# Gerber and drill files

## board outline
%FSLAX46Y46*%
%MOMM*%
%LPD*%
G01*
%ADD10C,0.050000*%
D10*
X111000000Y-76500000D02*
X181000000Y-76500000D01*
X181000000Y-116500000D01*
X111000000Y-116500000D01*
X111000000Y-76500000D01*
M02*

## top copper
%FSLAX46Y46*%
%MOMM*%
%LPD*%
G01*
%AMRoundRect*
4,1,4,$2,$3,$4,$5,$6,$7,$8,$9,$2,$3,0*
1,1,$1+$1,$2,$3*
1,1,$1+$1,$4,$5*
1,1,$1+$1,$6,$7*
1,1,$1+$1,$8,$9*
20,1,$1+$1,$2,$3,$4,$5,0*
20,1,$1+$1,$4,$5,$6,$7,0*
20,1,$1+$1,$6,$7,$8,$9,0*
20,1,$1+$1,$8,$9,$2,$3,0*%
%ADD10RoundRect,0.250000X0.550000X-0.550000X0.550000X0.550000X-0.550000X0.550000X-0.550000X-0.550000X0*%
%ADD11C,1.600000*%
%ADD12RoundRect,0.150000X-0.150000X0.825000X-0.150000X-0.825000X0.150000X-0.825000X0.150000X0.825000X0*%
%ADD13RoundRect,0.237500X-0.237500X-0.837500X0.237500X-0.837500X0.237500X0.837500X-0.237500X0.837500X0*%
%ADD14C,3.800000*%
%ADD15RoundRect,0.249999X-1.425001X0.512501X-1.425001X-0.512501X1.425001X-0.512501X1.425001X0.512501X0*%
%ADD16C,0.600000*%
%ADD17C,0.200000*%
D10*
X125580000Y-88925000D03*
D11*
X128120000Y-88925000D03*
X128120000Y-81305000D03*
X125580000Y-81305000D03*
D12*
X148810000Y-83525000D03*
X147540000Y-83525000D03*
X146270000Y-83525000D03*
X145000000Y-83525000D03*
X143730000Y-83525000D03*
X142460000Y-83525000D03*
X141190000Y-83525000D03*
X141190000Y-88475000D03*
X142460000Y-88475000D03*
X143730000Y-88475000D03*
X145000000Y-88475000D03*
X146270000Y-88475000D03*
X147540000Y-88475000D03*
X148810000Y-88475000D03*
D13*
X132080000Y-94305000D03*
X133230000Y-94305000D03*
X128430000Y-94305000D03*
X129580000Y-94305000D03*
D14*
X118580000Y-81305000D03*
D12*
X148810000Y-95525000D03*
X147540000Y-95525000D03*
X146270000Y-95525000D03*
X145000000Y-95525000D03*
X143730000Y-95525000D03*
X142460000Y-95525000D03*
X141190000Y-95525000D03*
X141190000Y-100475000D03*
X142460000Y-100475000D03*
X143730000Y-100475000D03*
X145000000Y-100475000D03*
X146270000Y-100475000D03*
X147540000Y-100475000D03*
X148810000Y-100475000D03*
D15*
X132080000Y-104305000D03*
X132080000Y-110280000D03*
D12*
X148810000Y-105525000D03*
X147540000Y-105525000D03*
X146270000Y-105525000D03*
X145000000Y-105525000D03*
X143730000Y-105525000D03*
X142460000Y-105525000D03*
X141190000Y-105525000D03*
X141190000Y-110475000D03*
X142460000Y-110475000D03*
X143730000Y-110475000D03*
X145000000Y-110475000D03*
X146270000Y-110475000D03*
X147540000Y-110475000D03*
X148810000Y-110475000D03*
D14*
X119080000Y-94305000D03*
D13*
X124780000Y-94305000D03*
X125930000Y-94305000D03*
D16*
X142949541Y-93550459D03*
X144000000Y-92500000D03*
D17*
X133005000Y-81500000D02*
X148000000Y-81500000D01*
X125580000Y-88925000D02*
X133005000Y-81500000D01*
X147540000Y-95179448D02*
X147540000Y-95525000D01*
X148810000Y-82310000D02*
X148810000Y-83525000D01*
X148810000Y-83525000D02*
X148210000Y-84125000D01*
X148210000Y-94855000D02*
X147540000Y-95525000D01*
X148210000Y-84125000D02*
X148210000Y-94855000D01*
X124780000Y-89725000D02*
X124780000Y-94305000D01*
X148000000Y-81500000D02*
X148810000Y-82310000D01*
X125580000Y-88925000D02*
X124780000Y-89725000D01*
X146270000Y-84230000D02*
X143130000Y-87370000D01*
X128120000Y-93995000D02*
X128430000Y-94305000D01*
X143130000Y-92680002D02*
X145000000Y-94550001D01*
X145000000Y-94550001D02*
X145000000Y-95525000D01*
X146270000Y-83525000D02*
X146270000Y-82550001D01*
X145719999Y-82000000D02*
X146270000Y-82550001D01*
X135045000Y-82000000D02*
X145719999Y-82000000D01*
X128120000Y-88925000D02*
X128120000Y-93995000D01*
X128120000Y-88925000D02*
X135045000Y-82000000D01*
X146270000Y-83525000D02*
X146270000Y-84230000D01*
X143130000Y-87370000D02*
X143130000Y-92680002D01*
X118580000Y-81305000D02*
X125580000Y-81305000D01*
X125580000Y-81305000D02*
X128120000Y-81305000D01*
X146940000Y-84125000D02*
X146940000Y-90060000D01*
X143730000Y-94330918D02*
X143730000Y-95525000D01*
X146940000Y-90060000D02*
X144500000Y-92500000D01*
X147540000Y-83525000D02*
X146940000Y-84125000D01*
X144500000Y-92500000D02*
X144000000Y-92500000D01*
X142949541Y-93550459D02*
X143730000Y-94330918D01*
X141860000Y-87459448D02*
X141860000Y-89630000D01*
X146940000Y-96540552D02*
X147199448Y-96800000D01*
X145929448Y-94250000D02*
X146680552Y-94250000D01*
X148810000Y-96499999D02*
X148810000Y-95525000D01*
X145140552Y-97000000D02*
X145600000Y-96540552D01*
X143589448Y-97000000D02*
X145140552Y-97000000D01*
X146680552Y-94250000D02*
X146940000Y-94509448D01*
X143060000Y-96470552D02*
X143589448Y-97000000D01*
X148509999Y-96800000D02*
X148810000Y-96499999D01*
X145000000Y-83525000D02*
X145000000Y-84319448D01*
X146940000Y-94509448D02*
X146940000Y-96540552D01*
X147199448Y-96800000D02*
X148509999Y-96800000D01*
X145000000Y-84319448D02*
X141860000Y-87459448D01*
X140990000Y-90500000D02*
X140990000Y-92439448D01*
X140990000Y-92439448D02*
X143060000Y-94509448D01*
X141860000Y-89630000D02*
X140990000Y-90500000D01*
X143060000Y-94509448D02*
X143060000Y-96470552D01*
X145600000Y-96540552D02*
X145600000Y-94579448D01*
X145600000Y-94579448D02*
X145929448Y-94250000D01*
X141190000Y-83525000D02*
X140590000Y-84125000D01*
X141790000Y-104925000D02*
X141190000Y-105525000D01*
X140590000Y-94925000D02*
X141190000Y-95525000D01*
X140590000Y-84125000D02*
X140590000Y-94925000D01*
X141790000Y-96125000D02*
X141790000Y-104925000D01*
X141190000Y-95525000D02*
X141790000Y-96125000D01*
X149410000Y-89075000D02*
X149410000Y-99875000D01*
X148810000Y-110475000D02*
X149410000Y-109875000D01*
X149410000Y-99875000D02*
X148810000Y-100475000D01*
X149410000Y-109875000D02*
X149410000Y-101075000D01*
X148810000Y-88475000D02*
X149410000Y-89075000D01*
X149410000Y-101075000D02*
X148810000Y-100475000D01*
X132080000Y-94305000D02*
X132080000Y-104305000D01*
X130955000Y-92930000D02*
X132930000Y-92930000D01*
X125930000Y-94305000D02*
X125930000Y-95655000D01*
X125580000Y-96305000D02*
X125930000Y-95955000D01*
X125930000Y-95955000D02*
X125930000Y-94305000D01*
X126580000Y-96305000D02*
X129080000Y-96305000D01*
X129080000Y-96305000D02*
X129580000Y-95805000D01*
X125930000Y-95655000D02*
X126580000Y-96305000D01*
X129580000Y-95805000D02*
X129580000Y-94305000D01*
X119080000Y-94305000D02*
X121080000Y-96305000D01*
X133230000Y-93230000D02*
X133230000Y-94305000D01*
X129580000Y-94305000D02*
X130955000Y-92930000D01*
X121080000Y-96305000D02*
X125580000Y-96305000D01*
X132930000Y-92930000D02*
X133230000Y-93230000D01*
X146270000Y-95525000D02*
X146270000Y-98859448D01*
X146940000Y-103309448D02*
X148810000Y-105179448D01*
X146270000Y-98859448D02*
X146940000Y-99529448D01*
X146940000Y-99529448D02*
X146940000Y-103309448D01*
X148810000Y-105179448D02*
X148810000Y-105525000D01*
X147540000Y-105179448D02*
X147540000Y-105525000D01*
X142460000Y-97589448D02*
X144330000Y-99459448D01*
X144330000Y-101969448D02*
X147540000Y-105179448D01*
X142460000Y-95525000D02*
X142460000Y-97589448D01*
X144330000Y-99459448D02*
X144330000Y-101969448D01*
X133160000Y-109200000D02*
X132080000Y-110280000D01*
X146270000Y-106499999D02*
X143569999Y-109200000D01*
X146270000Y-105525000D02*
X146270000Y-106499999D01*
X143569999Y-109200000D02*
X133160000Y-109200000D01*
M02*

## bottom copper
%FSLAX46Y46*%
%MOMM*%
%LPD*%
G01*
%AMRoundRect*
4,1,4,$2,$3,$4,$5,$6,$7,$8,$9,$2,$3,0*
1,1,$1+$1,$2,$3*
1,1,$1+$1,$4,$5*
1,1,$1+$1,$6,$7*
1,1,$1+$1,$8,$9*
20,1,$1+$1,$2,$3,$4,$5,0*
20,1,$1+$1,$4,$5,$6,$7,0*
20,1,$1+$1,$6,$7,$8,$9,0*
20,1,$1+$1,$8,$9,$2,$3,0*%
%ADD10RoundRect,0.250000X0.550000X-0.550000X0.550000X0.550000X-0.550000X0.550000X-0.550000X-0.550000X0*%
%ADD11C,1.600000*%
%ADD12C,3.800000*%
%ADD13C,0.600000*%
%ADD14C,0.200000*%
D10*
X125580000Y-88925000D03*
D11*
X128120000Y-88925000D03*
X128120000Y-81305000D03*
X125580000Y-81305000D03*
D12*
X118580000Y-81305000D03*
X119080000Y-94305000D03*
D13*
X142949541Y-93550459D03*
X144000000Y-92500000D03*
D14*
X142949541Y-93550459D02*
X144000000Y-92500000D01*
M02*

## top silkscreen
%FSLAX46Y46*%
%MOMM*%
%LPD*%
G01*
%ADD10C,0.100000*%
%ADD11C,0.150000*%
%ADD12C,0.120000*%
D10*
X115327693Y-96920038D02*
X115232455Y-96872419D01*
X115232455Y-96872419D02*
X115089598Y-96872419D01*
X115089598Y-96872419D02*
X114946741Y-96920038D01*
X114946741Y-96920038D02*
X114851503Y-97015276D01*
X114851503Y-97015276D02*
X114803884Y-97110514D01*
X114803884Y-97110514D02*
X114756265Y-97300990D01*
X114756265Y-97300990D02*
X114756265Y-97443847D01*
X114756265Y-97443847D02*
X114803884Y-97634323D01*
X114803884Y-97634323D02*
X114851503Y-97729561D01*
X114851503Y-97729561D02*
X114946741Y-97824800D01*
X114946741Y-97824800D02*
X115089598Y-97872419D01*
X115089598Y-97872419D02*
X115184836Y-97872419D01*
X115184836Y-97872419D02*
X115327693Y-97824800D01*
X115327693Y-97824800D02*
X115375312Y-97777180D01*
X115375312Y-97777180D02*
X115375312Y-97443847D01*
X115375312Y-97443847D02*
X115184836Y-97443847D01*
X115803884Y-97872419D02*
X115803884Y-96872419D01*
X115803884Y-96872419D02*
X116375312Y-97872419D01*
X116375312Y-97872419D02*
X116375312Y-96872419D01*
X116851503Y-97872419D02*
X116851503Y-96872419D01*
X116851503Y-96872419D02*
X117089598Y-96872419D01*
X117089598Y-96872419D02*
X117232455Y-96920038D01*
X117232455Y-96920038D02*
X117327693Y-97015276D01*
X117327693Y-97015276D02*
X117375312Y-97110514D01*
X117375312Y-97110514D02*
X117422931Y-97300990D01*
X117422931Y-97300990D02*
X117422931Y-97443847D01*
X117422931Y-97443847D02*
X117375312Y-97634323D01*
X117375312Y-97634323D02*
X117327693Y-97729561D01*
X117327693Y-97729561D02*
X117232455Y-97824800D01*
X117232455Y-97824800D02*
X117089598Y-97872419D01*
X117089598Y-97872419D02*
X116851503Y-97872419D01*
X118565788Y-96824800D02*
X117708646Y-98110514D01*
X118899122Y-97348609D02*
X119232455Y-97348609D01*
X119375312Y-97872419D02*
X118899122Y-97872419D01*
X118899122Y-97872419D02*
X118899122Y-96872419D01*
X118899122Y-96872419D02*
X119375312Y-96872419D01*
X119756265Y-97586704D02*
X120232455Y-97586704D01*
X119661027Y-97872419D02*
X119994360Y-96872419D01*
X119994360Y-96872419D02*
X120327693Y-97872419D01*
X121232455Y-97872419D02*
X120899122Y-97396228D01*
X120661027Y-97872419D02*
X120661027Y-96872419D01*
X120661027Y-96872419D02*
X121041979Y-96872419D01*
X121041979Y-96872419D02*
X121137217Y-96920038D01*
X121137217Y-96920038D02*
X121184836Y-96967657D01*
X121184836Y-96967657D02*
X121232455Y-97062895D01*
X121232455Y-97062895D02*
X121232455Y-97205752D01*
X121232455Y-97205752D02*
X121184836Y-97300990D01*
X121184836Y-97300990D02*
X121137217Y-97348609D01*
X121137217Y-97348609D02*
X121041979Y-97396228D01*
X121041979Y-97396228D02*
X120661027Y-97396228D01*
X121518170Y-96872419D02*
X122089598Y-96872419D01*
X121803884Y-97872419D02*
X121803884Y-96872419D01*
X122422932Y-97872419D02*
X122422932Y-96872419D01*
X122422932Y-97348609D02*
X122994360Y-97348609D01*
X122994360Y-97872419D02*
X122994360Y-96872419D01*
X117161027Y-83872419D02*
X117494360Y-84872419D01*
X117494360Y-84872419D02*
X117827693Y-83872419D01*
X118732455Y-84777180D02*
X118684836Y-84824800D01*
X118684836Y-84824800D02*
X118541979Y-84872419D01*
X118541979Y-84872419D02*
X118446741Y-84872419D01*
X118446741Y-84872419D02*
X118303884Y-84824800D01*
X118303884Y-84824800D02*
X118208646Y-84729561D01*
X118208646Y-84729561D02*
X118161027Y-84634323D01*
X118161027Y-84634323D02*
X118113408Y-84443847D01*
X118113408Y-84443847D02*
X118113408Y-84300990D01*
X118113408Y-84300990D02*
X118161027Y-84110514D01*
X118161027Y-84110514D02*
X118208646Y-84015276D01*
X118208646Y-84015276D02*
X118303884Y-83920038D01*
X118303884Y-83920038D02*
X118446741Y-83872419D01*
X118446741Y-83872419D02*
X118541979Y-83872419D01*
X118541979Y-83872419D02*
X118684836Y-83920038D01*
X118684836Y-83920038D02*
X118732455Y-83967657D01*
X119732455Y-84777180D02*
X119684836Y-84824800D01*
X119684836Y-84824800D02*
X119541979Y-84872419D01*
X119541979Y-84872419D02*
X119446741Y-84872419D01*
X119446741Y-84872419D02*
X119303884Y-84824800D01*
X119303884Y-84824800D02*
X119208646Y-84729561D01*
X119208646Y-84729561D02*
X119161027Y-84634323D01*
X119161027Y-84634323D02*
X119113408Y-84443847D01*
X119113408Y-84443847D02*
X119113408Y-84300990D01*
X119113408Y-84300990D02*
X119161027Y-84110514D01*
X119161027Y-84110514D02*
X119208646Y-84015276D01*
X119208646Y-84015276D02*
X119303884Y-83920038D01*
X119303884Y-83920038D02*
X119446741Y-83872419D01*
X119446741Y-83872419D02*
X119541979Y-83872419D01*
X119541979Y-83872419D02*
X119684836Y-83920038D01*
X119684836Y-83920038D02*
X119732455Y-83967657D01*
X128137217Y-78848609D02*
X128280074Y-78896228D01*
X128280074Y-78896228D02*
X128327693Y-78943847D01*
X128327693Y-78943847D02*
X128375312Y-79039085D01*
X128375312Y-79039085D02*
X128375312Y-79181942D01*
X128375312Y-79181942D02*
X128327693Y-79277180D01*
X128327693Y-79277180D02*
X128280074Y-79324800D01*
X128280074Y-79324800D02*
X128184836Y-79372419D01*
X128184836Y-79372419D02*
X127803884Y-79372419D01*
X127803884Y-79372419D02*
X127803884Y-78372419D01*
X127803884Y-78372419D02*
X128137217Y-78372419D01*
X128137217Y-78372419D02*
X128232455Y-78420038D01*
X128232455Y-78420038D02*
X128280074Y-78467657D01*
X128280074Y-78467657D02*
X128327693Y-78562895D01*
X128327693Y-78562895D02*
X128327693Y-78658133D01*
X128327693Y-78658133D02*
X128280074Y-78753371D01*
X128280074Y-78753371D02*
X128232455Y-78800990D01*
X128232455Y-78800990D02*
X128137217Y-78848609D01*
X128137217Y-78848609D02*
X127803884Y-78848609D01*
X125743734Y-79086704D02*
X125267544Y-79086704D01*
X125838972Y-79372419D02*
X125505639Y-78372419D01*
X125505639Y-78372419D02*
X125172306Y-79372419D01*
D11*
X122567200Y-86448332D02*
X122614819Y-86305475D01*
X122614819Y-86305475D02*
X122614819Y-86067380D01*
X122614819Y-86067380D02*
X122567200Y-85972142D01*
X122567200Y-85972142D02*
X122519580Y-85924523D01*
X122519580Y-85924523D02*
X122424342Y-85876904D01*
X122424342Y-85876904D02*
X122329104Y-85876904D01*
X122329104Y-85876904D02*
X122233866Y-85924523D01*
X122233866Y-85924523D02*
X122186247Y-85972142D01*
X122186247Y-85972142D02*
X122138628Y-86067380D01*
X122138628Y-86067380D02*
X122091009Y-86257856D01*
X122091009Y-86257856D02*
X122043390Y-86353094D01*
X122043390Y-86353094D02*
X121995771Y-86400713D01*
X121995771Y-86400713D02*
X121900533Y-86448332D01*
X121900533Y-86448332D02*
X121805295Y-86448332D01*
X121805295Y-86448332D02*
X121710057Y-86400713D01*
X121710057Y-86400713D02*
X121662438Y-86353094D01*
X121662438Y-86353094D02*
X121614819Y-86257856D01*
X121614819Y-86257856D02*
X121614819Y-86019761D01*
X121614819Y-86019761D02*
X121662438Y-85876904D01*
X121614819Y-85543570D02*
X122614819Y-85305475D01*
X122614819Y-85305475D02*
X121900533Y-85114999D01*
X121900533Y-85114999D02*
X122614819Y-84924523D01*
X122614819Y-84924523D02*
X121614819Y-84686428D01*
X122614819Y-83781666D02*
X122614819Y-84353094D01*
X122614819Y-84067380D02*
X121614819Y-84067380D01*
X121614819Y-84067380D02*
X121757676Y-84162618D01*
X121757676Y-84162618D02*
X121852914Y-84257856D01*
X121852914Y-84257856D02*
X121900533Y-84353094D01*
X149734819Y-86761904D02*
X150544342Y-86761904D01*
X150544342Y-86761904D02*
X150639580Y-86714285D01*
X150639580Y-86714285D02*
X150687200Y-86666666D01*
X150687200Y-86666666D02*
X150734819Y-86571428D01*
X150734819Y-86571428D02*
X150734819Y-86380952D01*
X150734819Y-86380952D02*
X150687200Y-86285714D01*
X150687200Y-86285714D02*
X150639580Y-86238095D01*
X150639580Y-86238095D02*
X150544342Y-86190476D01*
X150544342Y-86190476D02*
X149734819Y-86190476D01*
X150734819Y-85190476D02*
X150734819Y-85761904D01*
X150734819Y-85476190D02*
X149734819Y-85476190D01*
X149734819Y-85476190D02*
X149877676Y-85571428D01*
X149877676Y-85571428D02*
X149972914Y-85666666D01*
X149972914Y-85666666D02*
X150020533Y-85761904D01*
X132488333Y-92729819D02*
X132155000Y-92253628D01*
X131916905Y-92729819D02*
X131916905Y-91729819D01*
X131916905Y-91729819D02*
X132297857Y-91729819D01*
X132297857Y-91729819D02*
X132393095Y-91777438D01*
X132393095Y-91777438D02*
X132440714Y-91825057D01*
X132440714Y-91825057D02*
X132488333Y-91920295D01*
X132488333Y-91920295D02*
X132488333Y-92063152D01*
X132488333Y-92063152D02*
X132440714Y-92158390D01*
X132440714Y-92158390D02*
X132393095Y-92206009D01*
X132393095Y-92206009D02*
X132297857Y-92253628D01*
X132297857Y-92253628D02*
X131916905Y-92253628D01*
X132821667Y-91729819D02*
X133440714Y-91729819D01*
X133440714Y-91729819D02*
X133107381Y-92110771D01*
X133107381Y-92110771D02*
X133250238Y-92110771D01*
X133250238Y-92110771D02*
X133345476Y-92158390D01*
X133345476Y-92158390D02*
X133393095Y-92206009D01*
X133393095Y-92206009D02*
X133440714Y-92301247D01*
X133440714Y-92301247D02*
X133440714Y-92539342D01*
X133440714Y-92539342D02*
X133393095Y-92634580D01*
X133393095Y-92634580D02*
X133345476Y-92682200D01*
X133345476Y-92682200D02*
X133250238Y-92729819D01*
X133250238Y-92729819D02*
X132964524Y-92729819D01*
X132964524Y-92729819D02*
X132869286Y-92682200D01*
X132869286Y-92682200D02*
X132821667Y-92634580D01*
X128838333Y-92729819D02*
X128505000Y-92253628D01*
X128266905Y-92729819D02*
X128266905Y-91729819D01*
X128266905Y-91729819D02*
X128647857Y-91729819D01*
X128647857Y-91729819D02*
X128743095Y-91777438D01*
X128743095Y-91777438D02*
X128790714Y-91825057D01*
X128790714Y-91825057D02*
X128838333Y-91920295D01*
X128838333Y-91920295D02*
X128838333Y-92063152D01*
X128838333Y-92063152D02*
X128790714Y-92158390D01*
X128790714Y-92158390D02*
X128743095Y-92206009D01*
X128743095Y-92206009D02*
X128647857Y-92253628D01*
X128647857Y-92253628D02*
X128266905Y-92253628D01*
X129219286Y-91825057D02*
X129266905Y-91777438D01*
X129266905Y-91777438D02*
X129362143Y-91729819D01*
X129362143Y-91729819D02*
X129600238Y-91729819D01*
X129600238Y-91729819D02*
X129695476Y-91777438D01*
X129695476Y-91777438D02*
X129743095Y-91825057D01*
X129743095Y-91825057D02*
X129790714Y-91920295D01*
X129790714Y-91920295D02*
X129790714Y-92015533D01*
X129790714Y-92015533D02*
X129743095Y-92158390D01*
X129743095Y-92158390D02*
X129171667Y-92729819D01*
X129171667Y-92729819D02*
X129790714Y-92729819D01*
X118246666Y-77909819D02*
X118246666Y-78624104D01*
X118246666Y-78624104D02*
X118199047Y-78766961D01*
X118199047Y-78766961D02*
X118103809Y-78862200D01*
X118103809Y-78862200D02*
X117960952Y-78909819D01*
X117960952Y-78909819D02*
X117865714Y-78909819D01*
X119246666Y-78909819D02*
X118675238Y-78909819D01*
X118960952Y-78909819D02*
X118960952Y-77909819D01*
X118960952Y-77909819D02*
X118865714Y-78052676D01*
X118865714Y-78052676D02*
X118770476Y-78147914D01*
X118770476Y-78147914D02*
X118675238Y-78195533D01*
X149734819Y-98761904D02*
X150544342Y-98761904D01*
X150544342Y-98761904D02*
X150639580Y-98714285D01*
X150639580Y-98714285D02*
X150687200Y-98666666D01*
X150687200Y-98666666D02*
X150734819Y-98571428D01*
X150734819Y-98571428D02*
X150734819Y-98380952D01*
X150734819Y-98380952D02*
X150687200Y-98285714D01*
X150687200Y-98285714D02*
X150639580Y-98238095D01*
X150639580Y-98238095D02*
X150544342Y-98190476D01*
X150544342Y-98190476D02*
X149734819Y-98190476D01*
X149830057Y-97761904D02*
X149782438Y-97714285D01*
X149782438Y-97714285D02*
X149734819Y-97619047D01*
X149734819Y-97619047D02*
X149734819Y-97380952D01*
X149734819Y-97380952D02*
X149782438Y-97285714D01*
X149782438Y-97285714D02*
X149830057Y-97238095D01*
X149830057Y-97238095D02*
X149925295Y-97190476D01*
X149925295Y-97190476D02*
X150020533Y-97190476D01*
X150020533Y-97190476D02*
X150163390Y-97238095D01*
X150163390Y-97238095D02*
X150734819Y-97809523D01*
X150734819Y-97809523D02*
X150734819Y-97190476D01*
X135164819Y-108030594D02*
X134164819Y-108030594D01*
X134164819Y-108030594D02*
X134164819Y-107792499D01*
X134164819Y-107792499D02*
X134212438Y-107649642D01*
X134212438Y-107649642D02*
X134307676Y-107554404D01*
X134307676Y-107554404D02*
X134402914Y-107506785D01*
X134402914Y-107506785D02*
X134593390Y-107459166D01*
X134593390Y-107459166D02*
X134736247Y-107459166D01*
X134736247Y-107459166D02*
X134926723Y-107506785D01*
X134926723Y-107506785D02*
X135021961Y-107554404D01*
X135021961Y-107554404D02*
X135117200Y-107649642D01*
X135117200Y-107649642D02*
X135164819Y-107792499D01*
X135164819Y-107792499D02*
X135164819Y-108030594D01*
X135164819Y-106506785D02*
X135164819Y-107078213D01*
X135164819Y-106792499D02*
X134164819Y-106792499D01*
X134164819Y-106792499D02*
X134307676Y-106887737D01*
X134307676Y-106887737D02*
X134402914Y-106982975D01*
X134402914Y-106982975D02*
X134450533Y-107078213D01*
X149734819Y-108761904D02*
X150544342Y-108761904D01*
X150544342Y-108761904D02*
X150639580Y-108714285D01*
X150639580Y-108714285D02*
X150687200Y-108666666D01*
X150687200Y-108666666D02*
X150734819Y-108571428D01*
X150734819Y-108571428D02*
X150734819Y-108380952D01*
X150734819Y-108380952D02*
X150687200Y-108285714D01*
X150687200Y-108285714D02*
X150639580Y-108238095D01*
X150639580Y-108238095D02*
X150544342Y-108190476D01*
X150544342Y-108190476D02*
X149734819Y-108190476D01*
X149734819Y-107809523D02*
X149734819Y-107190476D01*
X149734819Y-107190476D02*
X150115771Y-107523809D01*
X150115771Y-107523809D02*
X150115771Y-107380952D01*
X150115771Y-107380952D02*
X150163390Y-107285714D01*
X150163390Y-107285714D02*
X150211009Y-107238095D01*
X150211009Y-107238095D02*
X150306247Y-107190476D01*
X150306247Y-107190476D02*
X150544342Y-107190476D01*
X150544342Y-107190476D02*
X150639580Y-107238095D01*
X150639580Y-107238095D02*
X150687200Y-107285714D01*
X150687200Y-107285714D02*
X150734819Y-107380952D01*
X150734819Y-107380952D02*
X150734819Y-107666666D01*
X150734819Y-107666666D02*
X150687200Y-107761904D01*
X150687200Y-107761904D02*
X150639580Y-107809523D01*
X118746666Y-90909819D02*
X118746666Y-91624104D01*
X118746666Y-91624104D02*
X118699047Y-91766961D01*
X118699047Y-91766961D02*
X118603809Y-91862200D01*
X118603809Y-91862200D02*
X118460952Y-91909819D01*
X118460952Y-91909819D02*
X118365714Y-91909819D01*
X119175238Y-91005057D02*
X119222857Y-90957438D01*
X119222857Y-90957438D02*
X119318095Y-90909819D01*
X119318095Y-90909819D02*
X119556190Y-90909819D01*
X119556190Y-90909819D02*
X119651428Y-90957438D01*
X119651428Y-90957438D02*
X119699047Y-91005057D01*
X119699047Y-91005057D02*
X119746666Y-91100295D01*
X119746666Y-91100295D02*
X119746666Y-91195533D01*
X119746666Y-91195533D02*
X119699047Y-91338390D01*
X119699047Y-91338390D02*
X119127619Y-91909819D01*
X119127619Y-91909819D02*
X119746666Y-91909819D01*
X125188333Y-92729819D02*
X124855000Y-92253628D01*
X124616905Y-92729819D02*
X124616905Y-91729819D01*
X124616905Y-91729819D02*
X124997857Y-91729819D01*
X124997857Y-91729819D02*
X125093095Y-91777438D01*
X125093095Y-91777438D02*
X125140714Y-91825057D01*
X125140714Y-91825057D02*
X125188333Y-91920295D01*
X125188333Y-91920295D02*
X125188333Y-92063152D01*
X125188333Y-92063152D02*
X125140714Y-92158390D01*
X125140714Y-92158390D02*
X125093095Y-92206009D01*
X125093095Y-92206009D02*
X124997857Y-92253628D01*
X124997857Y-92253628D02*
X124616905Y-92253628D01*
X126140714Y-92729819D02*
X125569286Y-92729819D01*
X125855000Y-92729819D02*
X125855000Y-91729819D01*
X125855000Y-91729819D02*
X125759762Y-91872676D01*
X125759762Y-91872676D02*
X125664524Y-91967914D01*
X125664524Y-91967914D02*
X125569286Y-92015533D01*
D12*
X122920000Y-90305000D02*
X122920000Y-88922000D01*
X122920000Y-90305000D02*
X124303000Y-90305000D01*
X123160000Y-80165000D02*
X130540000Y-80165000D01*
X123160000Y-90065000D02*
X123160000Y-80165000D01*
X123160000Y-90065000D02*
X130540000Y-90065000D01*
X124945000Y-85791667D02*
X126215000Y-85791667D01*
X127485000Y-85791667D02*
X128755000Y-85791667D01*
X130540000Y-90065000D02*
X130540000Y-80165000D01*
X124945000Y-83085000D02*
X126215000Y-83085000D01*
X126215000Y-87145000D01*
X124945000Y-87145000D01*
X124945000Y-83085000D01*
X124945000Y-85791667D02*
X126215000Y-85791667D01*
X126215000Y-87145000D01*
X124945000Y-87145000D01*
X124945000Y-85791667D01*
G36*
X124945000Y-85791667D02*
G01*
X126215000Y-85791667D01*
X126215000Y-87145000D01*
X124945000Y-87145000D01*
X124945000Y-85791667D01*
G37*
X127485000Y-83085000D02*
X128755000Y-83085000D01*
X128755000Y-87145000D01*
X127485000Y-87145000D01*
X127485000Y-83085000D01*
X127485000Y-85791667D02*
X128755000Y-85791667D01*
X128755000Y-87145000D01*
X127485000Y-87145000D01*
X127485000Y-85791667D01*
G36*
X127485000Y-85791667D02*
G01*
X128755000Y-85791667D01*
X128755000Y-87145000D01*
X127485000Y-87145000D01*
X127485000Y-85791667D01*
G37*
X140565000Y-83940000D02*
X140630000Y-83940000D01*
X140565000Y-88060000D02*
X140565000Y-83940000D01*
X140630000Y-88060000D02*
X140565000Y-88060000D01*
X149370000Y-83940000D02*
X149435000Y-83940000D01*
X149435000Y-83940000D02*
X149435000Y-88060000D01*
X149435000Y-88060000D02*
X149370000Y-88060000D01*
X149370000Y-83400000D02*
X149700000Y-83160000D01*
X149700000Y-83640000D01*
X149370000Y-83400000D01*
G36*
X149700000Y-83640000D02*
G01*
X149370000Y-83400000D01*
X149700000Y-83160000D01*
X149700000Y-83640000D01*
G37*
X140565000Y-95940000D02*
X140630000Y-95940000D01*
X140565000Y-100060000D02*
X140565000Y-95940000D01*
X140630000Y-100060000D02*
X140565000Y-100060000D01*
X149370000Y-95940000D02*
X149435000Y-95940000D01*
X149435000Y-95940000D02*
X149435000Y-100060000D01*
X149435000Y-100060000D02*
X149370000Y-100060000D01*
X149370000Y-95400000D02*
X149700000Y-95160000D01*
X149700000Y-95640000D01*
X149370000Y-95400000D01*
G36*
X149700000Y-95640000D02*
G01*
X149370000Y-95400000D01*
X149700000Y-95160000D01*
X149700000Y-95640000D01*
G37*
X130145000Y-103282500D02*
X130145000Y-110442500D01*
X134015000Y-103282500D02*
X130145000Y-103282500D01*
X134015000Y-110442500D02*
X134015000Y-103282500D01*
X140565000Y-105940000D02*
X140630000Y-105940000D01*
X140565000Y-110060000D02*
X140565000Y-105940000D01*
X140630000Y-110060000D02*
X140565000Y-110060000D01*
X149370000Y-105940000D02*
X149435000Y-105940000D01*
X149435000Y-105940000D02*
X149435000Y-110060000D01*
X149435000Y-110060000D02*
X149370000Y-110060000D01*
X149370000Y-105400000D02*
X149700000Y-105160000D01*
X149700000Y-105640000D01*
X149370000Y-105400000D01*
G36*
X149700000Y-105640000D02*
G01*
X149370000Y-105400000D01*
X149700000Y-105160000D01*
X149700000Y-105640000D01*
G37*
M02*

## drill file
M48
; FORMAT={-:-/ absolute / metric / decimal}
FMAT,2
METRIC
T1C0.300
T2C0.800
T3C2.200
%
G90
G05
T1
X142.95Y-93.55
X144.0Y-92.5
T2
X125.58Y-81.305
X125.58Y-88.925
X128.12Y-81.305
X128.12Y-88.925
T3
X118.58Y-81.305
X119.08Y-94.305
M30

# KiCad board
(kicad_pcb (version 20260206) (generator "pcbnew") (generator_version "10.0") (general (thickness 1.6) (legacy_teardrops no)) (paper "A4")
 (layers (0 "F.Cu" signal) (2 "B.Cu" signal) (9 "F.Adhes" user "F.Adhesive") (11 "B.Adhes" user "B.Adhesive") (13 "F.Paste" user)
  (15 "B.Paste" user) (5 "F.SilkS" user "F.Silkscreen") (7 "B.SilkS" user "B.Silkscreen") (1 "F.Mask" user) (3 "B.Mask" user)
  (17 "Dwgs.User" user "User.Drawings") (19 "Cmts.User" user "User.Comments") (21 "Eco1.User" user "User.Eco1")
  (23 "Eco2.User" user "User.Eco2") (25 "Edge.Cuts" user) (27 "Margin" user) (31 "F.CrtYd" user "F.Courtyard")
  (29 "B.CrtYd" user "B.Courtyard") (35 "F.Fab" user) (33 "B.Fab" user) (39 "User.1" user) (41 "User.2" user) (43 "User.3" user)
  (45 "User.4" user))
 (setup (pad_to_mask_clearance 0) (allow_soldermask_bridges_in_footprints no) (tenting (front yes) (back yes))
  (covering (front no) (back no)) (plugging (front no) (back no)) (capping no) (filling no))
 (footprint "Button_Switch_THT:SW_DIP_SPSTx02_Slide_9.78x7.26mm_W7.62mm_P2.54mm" (layer "F.Cu") (at 125.58 88.925 90)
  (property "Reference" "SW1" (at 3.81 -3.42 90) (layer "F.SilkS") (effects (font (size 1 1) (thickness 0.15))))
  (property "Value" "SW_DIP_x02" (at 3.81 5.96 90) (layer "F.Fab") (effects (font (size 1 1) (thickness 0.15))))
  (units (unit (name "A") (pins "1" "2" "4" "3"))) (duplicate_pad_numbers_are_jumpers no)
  (fp_line (start -1.38 -2.66) (end 0.003 -2.66) (stroke (width 0.12) (type solid)) (layer "F.SilkS"))
  (fp_line (start -1.38 -2.66) (end -1.38 -1.277) (stroke (width 0.12) (type solid)) (layer "F.SilkS"))
  (fp_line (start 8.76 -2.42) (end 8.76 4.96) (stroke (width 0.12) (type solid)) (layer "F.SilkS"))
  (fp_line (start -1.14 -2.42) (end 8.76 -2.42) (stroke (width 0.12) (type solid)) (layer "F.SilkS"))
  (fp_line (start -1.14 -2.42) (end -1.14 4.96) (stroke (width 0.12) (type solid)) (layer "F.SilkS"))
  (fp_line (start 3.133333 -0.635) (end 3.133333 0.635) (stroke (width 0.12) (type solid)) (layer "F.SilkS"))
  (fp_line (start 3.133333 1.905) (end 3.133333 3.175) (stroke (width 0.12) (type solid)) (layer "F.SilkS"))
  (fp_line (start -1.14 4.96) (end 8.76 4.96) (stroke (width 0.12) (type solid)) (layer "F.SilkS"))
  (fp_rect (start 1.78 -0.635) (end 5.84 0.635) (stroke (width 0.12) (type solid)) (fill no) (layer "F.SilkS"))
  (fp_rect (start 1.78 -0.635) (end 3.133333 0.635) (stroke (width 0.12) (type solid)) (fill yes) (layer "F.SilkS"))
  (fp_rect (start 1.78 1.905) (end 5.84 3.175) (stroke (width 0.12) (type solid)) (fill no) (layer "F.SilkS"))
  (fp_rect (start 1.78 1.905) (end 3.133333 3.175) (stroke (width 0.12) (type solid)) (fill yes) (layer "F.SilkS"))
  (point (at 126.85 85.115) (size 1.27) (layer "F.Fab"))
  (pad "1" thru_hole roundrect (at 0 0 90) (size 1.6 1.6) (drill 0.8) (layers "*.Cu" "*.Mask") (remove_unused_layers no)
   (roundrect_rratio 0.15625) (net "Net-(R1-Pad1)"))
  (pad "2" thru_hole circle (at 0 2.54 90) (size 1.6 1.6) (drill 0.8) (layers "*.Cu" "*.Mask") (remove_unused_layers no)
   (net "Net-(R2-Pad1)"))
  (pad "3" thru_hole circle (at 7.62 2.54 90) (size 1.6 1.6) (drill 0.8) (layers "*.Cu" "*.Mask") (remove_unused_layers no) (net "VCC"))
  (pad "4" thru_hole circle (at 7.62 0 90) (size 1.6 1.6) (drill 0.8) (layers "*.Cu" "*.Mask") (remove_unused_layers no) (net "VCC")))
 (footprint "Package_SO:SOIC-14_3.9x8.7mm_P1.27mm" (layer "F.Cu") (at 145 86 -90)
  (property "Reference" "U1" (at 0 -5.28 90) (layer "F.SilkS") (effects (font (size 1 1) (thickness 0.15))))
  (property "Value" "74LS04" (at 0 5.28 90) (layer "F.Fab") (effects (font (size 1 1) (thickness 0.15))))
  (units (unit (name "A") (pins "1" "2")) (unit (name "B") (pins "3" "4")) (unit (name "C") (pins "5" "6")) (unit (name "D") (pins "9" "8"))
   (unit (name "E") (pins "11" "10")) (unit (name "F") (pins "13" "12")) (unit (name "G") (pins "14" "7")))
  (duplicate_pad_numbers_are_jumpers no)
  (fp_line (start -2.06 4.435) (end -2.06 4.37) (stroke (width 0.12) (type solid)) (layer "F.SilkS"))
  (fp_line (start 2.06 4.435) (end -2.06 4.435) (stroke (width 0.12) (type solid)) (layer "F.SilkS"))
  (fp_line (start 2.06 4.37) (end 2.06 4.435) (stroke (width 0.12) (type solid)) (layer "F.SilkS"))
  (fp_line (start -2.06 -4.37) (end -2.06 -4.435) (stroke (width 0.12) (type solid)) (layer "F.SilkS"))
  (fp_line (start -2.06 -4.435) (end 2.06 -4.435) (stroke (width 0.12) (type solid)) (layer "F.SilkS"))
  (fp_line (start 2.06 -4.435) (end 2.06 -4.37) (stroke (width 0.12) (type solid)) (layer "F.SilkS"))
  (fp_poly (pts (xy -2.6 -4.37) (xy -2.84 -4.7) (xy -2.36 -4.7)) (stroke (width 0.12) (type solid)) (fill yes) (layer "F.SilkS"))
  (pad "1" smd roundrect (at -2.475 -3.81 270) (size 1.95 0.6) (layers "F.Cu" "F.Mask" "F.Paste") (roundrect_rratio 0.25)
   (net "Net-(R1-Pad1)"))
  (pad "2" smd roundrect (at -2.475 -2.54 270) (size 1.95 0.6) (layers "F.Cu" "F.Mask" "F.Paste") (roundrect_rratio 0.25)
   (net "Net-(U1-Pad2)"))
  (pad "3" smd roundrect (at -2.475 -1.27 270) (size 1.95 0.6) (layers "F.Cu" "F.Mask" "F.Paste") (roundrect_rratio 0.25)
   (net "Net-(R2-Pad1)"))
  (pad "4" smd roundrect (at -2.475 0 270) (size 1.95 0.6) (layers "F.Cu" "F.Mask" "F.Paste") (roundrect_rratio 0.25) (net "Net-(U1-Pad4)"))
  (pad "5" smd roundrect (at -2.475 1.27 270) (size 1.95 0.6) (layers "F.Cu" "F.Mask" "F.Paste") (roundrect_rratio 0.25)
   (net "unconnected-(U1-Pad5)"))
  (pad "6" smd roundrect (at -2.475 2.54 270) (size 1.95 0.6) (layers "F.Cu" "F.Mask" "F.Paste") (roundrect_rratio 0.25)
   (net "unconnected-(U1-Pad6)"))
  (pad "7" smd roundrect (at -2.475 3.81 270) (size 1.95 0.6) (layers "F.Cu" "F.Mask" "F.Paste") (roundrect_rratio 0.25)
   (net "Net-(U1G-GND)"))
  (pad "8" smd roundrect (at 2.475 3.81 270) (size 1.95 0.6) (layers "F.Cu" "F.Mask" "F.Paste") (roundrect_rratio 0.25)
   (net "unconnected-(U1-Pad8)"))
  (pad "9" smd roundrect (at 2.475 2.54 270) (size 1.95 0.6) (layers "F.Cu" "F.Mask" "F.Paste") (roundrect_rratio 0.25)
   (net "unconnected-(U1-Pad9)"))
  (pad "10" smd roundrect (at 2.475 1.27 270) (size 1.95 0.6) (layers "F.Cu" "F.Mask" "F.Paste") (roundrect_rratio 0.25)
   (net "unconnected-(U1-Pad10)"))
  (pad "11" smd roundrect (at 2.475 0 270) (size 1.95 0.6) (layers "F.Cu" "F.Mask" "F.Paste") (roundrect_rratio 0.25)
   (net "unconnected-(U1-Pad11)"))
  (pad "12" smd roundrect (at 2.475 -1.27 270) (size 1.95 0.6) (layers "F.Cu" "F.Mask" "F.Paste") (roundrect_rratio 0.25)
   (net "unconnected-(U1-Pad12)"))
  (pad "13" smd roundrect (at 2.475 -2.54 270) (size 1.95 0.6) (layers "F.Cu" "F.Mask" "F.Paste") (roundrect_rratio 0.25)
   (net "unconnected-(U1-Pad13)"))
  (pad "14" smd roundrect (at 2.475 -3.81 270) (size 1.95 0.6) (layers "F.Cu" "F.Mask" "F.Paste") (roundrect_rratio 0.25)
   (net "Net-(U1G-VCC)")))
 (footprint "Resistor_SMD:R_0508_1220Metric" (layer "F.Cu") (at 132.655 94.305)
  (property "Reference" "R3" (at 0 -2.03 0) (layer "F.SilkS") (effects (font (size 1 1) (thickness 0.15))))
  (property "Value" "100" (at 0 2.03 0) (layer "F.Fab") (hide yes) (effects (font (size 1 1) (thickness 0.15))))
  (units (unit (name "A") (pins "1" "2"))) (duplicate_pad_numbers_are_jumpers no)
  (pad "1" smd roundrect (at -0.575 0) (size 0.95 2.15) (layers "F.Cu" "F.Mask" "F.Paste") (roundrect_rratio 0.25) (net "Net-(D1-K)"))
  (pad "2" smd roundrect (at 0.575 0) (size 0.95 2.15) (layers "F.Cu" "F.Mask" "F.Paste") (roundrect_rratio 0.25) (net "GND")))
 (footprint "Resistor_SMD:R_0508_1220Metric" (layer "F.Cu") (at 129.005 94.305)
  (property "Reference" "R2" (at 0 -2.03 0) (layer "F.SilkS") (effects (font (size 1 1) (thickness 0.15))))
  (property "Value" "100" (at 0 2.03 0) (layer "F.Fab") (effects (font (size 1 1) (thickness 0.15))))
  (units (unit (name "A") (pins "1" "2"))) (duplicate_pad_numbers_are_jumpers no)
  (pad "1" smd roundrect (at -0.575 0) (size 0.95 2.15) (layers "F.Cu" "F.Mask" "F.Paste") (roundrect_rratio 0.25) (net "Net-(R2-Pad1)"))
  (pad "2" smd roundrect (at 0.575 0) (size 0.95 2.15) (layers "F.Cu" "F.Mask" "F.Paste") (roundrect_rratio 0.25) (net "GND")))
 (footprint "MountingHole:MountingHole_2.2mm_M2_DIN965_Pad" (layer "F.Cu") (at 118.58 81.305)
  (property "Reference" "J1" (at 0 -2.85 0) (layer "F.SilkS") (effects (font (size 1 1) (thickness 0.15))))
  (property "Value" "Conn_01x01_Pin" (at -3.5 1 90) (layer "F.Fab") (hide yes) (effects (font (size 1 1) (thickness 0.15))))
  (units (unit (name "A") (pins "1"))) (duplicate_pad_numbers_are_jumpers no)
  (pad "1" thru_hole circle (at 0 0) (size 3.8 3.8) (drill 2.2) (layers "*.Cu" "*.Mask") (remove_unused_layers no) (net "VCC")
   (zone_connect 2)))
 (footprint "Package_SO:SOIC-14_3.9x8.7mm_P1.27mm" (layer "F.Cu") (at 145 98 -90)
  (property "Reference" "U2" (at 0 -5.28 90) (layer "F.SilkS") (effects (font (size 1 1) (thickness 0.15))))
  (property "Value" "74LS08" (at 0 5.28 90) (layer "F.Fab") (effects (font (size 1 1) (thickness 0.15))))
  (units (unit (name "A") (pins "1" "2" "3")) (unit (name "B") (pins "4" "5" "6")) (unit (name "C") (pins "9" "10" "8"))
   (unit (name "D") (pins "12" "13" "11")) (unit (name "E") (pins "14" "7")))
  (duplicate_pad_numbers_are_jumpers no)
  (fp_line (start -2.06 4.435) (end -2.06 4.37) (stroke (width 0.12) (type solid)) (layer "F.SilkS"))
  (fp_line (start 2.06 4.435) (end -2.06 4.435) (stroke (width 0.12) (type solid)) (layer "F.SilkS"))
  (fp_line (start 2.06 4.37) (end 2.06 4.435) (stroke (width 0.12) (type solid)) (layer "F.SilkS"))
  (fp_line (start -2.06 -4.37) (end -2.06 -4.435) (stroke (width 0.12) (type solid)) (layer "F.SilkS"))
  (fp_line (start -2.06 -4.435) (end 2.06 -4.435) (stroke (width 0.12) (type solid)) (layer "F.SilkS"))
  (fp_line (start 2.06 -4.435) (end 2.06 -4.37) (stroke (width 0.12) (type solid)) (layer "F.SilkS"))
  (fp_poly (pts (xy -2.6 -4.37) (xy -2.84 -4.7) (xy -2.36 -4.7)) (stroke (width 0.12) (type solid)) (fill yes) (layer "F.SilkS"))
  (pad "1" smd roundrect (at -2.475 -3.81 270) (size 1.95 0.6) (layers "F.Cu" "F.Mask" "F.Paste") (roundrect_rratio 0.25)
   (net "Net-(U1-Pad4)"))
  (pad "2" smd roundrect (at -2.475 -2.54 270) (size 1.95 0.6) (layers "F.Cu" "F.Mask" "F.Paste") (roundrect_rratio 0.25)
   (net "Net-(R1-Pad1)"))
  (pad "3" smd roundrect (at -2.475 -1.27 270) (size 1.95 0.6) (layers "F.Cu" "F.Mask" "F.Paste") (roundrect_rratio 0.25)
   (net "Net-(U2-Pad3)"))
  (pad "4" smd roundrect (at -2.475 0 270) (size 1.95 0.6) (layers "F.Cu" "F.Mask" "F.Paste") (roundrect_rratio 0.25) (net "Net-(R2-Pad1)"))
  (pad "5" smd roundrect (at -2.475 1.27 270) (size 1.95 0.6) (layers "F.Cu" "F.Mask" "F.Paste") (roundrect_rratio 0.25)
   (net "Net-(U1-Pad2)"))
  (pad "6" smd roundrect (at -2.475 2.54 270) (size 1.95 0.6) (layers "F.Cu" "F.Mask" "F.Paste") (roundrect_rratio 0.25)
   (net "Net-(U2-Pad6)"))
  (pad "7" smd roundrect (at -2.475 3.81 270) (size 1.95 0.6) (layers "F.Cu" "F.Mask" "F.Paste") (roundrect_rratio 0.25)
   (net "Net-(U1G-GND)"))
  (pad "8" smd roundrect (at 2.475 3.81 270) (size 1.95 0.6) (layers "F.Cu" "F.Mask" "F.Paste") (roundrect_rratio 0.25)
   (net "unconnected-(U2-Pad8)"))
  (pad "9" smd roundrect (at 2.475 2.54 270) (size 1.95 0.6) (layers "F.Cu" "F.Mask" "F.Paste") (roundrect_rratio 0.25)
   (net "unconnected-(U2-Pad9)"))
  (pad "10" smd roundrect (at 2.475 1.27 270) (size 1.95 0.6) (layers "F.Cu" "F.Mask" "F.Paste") (roundrect_rratio 0.25)
   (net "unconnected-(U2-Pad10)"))
  (pad "11" smd roundrect (at 2.475 0 270) (size 1.95 0.6) (layers "F.Cu" "F.Mask" "F.Paste") (roundrect_rratio 0.25)
   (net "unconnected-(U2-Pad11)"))
  (pad "12" smd roundrect (at 2.475 -1.27 270) (size 1.95 0.6) (layers "F.Cu" "F.Mask" "F.Paste") (roundrect_rratio 0.25)
   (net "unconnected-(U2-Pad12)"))
  (pad "13" smd roundrect (at 2.475 -2.54 270) (size 1.95 0.6) (layers "F.Cu" "F.Mask" "F.Paste") (roundrect_rratio 0.25)
   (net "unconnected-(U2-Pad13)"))
  (pad "14" smd roundrect (at 2.475 -3.81 270) (size 1.95 0.6) (layers "F.Cu" "F.Mask" "F.Paste") (roundrect_rratio 0.25)
   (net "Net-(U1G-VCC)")))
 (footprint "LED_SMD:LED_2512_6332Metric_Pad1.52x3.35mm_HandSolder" (layer "F.Cu") (at 132.08 107.2925 -90)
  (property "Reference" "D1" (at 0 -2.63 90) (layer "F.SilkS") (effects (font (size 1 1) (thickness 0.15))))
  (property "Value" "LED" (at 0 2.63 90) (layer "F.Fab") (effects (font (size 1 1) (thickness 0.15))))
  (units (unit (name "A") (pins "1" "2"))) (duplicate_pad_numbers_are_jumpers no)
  (fp_line (start -4.01 1.935) (end 3.15 1.935) (stroke (width 0.12) (type solid)) (layer "F.SilkS"))
  (fp_line (start -4.01 -1.935) (end -4.01 1.935) (stroke (width 0.12) (type solid)) (layer "F.SilkS"))
  (fp_line (start 3.15 -1.935) (end -4.01 -1.935) (stroke (width 0.12) (type solid)) (layer "F.SilkS"))
  (pad "1" smd roundrect (at -2.9875 0 270) (size 1.525 3.35) (layers "F.Cu" "F.Mask" "F.Paste") (roundrect_rratio 0.163934)
   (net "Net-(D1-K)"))
  (pad "2" smd roundrect (at 2.9875 0 270) (size 1.525 3.35) (layers "F.Cu" "F.Mask" "F.Paste") (roundrect_rratio 0.163934)
   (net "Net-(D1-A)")))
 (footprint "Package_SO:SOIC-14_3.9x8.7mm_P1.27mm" (layer "F.Cu") (at 145 108 -90)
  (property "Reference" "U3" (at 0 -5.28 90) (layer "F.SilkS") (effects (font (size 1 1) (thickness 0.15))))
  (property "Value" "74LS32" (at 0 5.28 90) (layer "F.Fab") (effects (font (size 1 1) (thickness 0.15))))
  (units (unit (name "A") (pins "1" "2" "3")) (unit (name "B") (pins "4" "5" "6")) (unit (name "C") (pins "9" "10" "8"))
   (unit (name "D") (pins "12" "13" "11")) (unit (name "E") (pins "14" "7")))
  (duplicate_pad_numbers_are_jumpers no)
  (fp_line (start -2.06 4.435) (end -2.06 4.37) (stroke (width 0.12) (type solid)) (layer "F.SilkS"))
  (fp_line (start 2.06 4.435) (end -2.06 4.435) (stroke (width 0.12) (type solid)) (layer "F.SilkS"))
  (fp_line (start 2.06 4.37) (end 2.06 4.435) (stroke (width 0.12) (type solid)) (layer "F.SilkS"))
  (fp_line (start -2.06 -4.37) (end -2.06 -4.435) (stroke (width 0.12) (type solid)) (layer "F.SilkS"))
  (fp_line (start -2.06 -4.435) (end 2.06 -4.435) (stroke (width 0.12) (type solid)) (layer "F.SilkS"))
  (fp_line (start 2.06 -4.435) (end 2.06 -4.37) (stroke (width 0.12) (type solid)) (layer "F.SilkS"))
  (fp_poly (pts (xy -2.6 -4.37) (xy -2.84 -4.7) (xy -2.36 -4.7)) (stroke (width 0.12) (type solid)) (fill yes) (layer "F.SilkS"))
  (pad "1" smd roundrect (at -2.475 -3.81 270) (size 1.95 0.6) (layers "F.Cu" "F.Mask" "F.Paste") (roundrect_rratio 0.25)
   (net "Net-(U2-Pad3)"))
  (pad "2" smd roundrect (at -2.475 -2.54 270) (size 1.95 0.6) (layers "F.Cu" "F.Mask" "F.Paste") (roundrect_rratio 0.25)
   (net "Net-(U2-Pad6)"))
  (pad "3" smd roundrect (at -2.475 -1.27 270) (size 1.95 0.6) (layers "F.Cu" "F.Mask" "F.Paste") (roundrect_rratio 0.25) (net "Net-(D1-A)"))
  (pad "4" smd roundrect (at -2.475 0 270) (size 1.95 0.6) (layers "F.Cu" "F.Mask" "F.Paste") (roundrect_rratio 0.25)
   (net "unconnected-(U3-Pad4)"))
  (pad "5" smd roundrect (at -2.475 1.27 270) (size 1.95 0.6) (layers "F.Cu" "F.Mask" "F.Paste") (roundrect_rratio 0.25)
   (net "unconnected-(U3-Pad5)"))
  (pad "6" smd roundrect (at -2.475 2.54 270) (size 1.95 0.6) (layers "F.Cu" "F.Mask" "F.Paste") (roundrect_rratio 0.25)
   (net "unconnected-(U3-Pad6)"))
  (pad "7" smd roundrect (at -2.475 3.81 270) (size 1.95 0.6) (layers "F.Cu" "F.Mask" "F.Paste") (roundrect_rratio 0.25)
   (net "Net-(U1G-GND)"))
  (pad "8" smd roundrect (at 2.475 3.81 270) (size 1.95 0.6) (layers "F.Cu" "F.Mask" "F.Paste") (roundrect_rratio 0.25)
   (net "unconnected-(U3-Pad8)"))
  (pad "9" smd roundrect (at 2.475 2.54 270) (size 1.95 0.6) (layers "F.Cu" "F.Mask" "F.Paste") (roundrect_rratio 0.25)
   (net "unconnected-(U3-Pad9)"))
  (pad "10" smd roundrect (at 2.475 1.27 270) (size 1.95 0.6) (layers "F.Cu" "F.Mask" "F.Paste") (roundrect_rratio 0.25)
   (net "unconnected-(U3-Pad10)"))
  (pad "11" smd roundrect (at 2.475 0 270) (size 1.95 0.6) (layers "F.Cu" "F.Mask" "F.Paste") (roundrect_rratio 0.25)
   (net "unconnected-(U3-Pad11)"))
  (pad "12" smd roundrect (at 2.475 -1.27 270) (size 1.95 0.6) (layers "F.Cu" "F.Mask" "F.Paste") (roundrect_rratio 0.25)
   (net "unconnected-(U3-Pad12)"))
  (pad "13" smd roundrect (at 2.475 -2.54 270) (size 1.95 0.6) (layers "F.Cu" "F.Mask" "F.Paste") (roundrect_rratio 0.25)
   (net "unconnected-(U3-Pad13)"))
  (pad "14" smd roundrect (at 2.475 -3.81 270) (size 1.95 0.6) (layers "F.Cu" "F.Mask" "F.Paste") (roundrect_rratio 0.25)
   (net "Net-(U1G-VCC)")))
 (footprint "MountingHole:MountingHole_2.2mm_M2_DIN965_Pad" (layer "F.Cu") (at 119.08 94.305)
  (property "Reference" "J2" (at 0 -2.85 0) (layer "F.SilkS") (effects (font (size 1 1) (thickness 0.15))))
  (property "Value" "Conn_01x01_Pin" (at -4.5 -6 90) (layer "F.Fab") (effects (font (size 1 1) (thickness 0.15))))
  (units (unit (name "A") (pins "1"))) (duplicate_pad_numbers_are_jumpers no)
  (pad "1" thru_hole circle (at 0 0) (size 3.8 3.8) (drill 2.2) (layers "*.Cu" "*.Mask") (remove_unused_layers no) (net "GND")
   (zone_connect 2)))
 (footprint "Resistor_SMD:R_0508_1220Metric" (layer "F.Cu") (at 125.355 94.305)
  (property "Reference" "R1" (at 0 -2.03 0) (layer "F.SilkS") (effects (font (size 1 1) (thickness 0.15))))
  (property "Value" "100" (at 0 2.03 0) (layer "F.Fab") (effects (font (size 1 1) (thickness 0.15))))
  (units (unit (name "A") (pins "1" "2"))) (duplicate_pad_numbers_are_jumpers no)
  (pad "1" smd roundrect (at -0.575 0) (size 0.95 2.15) (layers "F.Cu" "F.Mask" "F.Paste") (roundrect_rratio 0.25) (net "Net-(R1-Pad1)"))
  (pad "2" smd roundrect (at 0.575 0) (size 0.95 2.15) (layers "F.Cu" "F.Mask" "F.Paste") (roundrect_rratio 0.25) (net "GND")))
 (gr_rect (start 111 76.5) (end 181 116.5) (stroke (width 0.05) (type default)) (fill no) (layer "Edge.Cuts"))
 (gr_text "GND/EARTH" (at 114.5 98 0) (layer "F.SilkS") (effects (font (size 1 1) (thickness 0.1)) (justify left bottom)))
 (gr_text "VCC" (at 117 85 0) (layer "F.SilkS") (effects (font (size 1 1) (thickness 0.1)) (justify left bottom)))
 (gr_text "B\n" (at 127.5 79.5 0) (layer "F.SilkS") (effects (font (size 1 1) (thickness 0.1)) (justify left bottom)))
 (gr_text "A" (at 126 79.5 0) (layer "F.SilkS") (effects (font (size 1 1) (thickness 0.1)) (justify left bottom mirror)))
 (segment (start 133.005 81.5) (end 148 81.5) (width 0.2) (layer "F.Cu") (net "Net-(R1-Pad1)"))
 (segment (start 125.58 88.925) (end 133.005 81.5) (width 0.2) (layer "F.Cu") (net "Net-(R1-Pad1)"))
 (segment (start 147.54 95.179448) (end 147.54 95.525) (width 0.2) (layer "F.Cu") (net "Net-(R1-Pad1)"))
 (segment (start 148.81 82.31) (end 148.81 83.525) (width 0.2) (layer "F.Cu") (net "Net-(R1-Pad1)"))
 (segment (start 148.81 83.525) (end 148.21 84.125) (width 0.2) (layer "F.Cu") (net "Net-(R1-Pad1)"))
 (segment (start 148.21 94.855) (end 147.54 95.525) (width 0.2) (layer "F.Cu") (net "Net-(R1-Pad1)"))
 (segment (start 148.21 84.125) (end 148.21 94.855) (width 0.2) (layer "F.Cu") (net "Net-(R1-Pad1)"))
 (segment (start 124.78 89.725) (end 124.78 94.305) (width 0.2) (layer "F.Cu") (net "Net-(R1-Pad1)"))
 (segment (start 148 81.5) (end 148.81 82.31) (width 0.2) (layer "F.Cu") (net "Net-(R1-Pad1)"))
 (segment (start 125.58 88.925) (end 124.78 89.725) (width 0.2) (layer "F.Cu") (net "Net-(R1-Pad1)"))
 (segment (start 146.27 84.23) (end 143.13 87.37) (width 0.2) (layer "F.Cu") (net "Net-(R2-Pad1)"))
 (segment (start 128.12 93.995) (end 128.43 94.305) (width 0.2) (layer "F.Cu") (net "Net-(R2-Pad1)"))
 (segment (start 143.13 92.680002) (end 145 94.550001) (width 0.2) (layer "F.Cu") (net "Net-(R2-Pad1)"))
 (segment (start 145 94.550001) (end 145 95.525) (width 0.2) (layer "F.Cu") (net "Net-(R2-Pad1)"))
 (segment (start 146.27 83.525) (end 146.27 82.550001) (width 0.2) (layer "F.Cu") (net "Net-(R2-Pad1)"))
 (segment (start 145.719999 82) (end 146.27 82.550001) (width 0.2) (layer "F.Cu") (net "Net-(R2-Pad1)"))
 (segment (start 135.045 82) (end 145.719999 82) (width 0.2) (layer "F.Cu") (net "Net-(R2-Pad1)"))
 (segment (start 128.12 88.925) (end 128.12 93.995) (width 0.2) (layer "F.Cu") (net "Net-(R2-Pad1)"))
 (segment (start 128.12 88.925) (end 135.045 82) (width 0.2) (layer "F.Cu") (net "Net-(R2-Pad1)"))
 (segment (start 146.27 83.525) (end 146.27 84.23) (width 0.2) (layer "F.Cu") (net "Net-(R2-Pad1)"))
 (segment (start 143.13 87.37) (end 143.13 92.680002) (width 0.2) (layer "F.Cu") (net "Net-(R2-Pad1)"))
 (segment (start 118.58 81.305) (end 125.58 81.305) (width 0.2) (layer "F.Cu") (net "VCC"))
 (segment (start 125.58 81.305) (end 128.12 81.305) (width 0.2) (layer "F.Cu") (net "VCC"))
 (segment (start 146.94 84.125) (end 146.94 90.06) (width 0.2) (layer "F.Cu") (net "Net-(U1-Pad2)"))
 (segment (start 143.73 94.330918) (end 143.73 95.525) (width 0.2) (layer "F.Cu") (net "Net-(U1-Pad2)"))
 (segment (start 146.94 90.06) (end 144.5 92.5) (width 0.2) (layer "F.Cu") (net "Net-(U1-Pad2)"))
 (segment (start 147.54 83.525) (end 146.94 84.125) (width 0.2) (layer "F.Cu") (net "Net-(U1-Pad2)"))
 (segment (start 144.5 92.5) (end 144 92.5) (width 0.2) (layer "F.Cu") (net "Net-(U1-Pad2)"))
 (segment (start 142.949541 93.550459) (end 143.73 94.330918) (width 0.2) (layer "F.Cu") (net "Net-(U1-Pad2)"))
 (via (at 142.949541 93.550459) (size 0.6) (drill 0.3) (layers "F.Cu" "B.Cu") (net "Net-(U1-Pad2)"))
 (via (at 144 92.5) (size 0.6) (drill 0.3) (layers "F.Cu" "B.Cu") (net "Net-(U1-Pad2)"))
 (segment (start 142.949541 93.550459) (end 144 92.5) (width 0.2) (layer "B.Cu") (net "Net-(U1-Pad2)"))
 (segment (start 141.86 87.459448) (end 141.86 89.63) (width 0.2) (layer "F.Cu") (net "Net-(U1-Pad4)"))
 (segment (start 146.94 96.540552) (end 147.199448 96.8) (width 0.2) (layer "F.Cu") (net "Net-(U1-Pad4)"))
 (segment (start 145.929448 94.25) (end 146.680552 94.25) (width 0.2) (layer "F.Cu") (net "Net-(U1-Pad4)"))
 (segment (start 148.81 96.499999) (end 148.81 95.525) (width 0.2) (layer "F.Cu") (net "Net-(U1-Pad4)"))
 (segment (start 145.140552 97) (end 145.6 96.540552) (width 0.2) (layer "F.Cu") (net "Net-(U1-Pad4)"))
 (segment (start 143.589448 97) (end 145.140552 97) (width 0.2) (layer "F.Cu") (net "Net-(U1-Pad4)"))
 (segment (start 146.680552 94.25) (end 146.94 94.509448) (width 0.2) (layer "F.Cu") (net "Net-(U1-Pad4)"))
 (segment (start 143.06 96.470552) (end 143.589448 97) (width 0.2) (layer "F.Cu") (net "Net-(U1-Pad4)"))
 (segment (start 148.509999 96.8) (end 148.81 96.499999) (width 0.2) (layer "F.Cu") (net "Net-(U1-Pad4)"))
 (segment (start 145 83.525) (end 145 84.319448) (width 0.2) (layer "F.Cu") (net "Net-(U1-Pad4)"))
 (segment (start 146.94 94.509448) (end 146.94 96.540552) (width 0.2) (layer "F.Cu") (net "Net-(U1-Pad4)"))
 (segment (start 147.199448 96.8) (end 148.509999 96.8) (width 0.2) (layer "F.Cu") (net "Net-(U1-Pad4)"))
 (segment (start 145 84.319448) (end 141.86 87.459448) (width 0.2) (layer "F.Cu") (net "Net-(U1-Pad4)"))
 (segment (start 140.99 90.5) (end 140.99 92.439448) (width 0.2) (layer "F.Cu") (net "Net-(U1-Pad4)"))
 (segment (start 140.99 92.439448) (end 143.06 94.509448) (width 0.2) (layer "F.Cu") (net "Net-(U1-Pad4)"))
 (segment (start 141.86 89.63) (end 140.99 90.5) (width 0.2) (layer "F.Cu") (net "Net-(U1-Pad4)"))
 (segment (start 143.06 94.509448) (end 143.06 96.470552) (width 0.2) (layer "F.Cu") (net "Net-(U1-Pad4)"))
 (segment (start 145.6 96.540552) (end 145.6 94.579448) (width 0.2) (layer "F.Cu") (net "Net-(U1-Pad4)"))
 (segment (start 145.6 94.579448) (end 145.929448 94.25) (width 0.2) (layer "F.Cu") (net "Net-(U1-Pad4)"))
 (segment (start 141.19 83.525) (end 140.59 84.125) (width 0.2) (layer "F.Cu") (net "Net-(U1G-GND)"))
 (segment (start 141.79 104.925) (end 141.19 105.525) (width 0.2) (layer "F.Cu") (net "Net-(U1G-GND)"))
 (segment (start 140.59 94.925) (end 141.19 95.525) (width 0.2) (layer "F.Cu") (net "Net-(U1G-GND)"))
 (segment (start 140.59 84.125) (end 140.59 94.925) (width 0.2) (layer "F.Cu") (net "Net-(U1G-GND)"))
 (segment (start 141.79 96.125) (end 141.79 104.925) (width 0.2) (layer "F.Cu") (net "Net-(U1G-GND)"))
 (segment (start 141.19 95.525) (end 141.79 96.125) (width 0.2) (layer "F.Cu") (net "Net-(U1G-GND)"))
 (segment (start 149.41 89.075) (end 149.41 99.875) (width 0.2) (layer "F.Cu") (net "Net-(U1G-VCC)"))
 (segment (start 148.81 110.475) (end 149.41 109.875) (width 0.2) (layer "F.Cu") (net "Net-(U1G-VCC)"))
 (segment (start 149.41 99.875) (end 148.81 100.475) (width 0.2) (layer "F.Cu") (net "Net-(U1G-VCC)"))
 (segment (start 149.41 109.875) (end 149.41 101.075) (width 0.2) (layer "F.Cu") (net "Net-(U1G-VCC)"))
 (segment (start 148.81 88.475) (end 149.41 89.075) (width 0.2) (layer "F.Cu") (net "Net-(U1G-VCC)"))
 (segment (start 149.41 101.075) (end 148.81 100.475) (width 0.2) (layer "F.Cu") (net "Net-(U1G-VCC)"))
 (segment (start 132.08 94.305) (end 132.08 104.305) (width 0.2) (layer "F.Cu") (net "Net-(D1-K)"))
 (segment (start 130.955 92.93) (end 132.93 92.93) (width 0.2) (layer "F.Cu") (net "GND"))
 (segment (start 125.93 94.305) (end 125.93 95.655) (width 0.2) (layer "F.Cu") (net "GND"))
 (segment (start 125.58 96.305) (end 125.93 95.955) (width 0.2) (layer "F.Cu") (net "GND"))
 (segment (start 125.93 95.955) (end 125.93 94.305) (width 0.2) (layer "F.Cu") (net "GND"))
 (segment (start 126.58 96.305) (end 129.08 96.305) (width 0.2) (layer "F.Cu") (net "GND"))
 (segment (start 129.08 96.305) (end 129.58 95.805) (width 0.2) (layer "F.Cu") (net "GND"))
 (segment (start 125.93 95.655) (end 126.58 96.305) (width 0.2) (layer "F.Cu") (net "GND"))
 (segment (start 129.58 95.805) (end 129.58 94.305) (width 0.2) (layer "F.Cu") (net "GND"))
 (segment (start 119.08 94.305) (end 121.08 96.305) (width 0.2) (layer "F.Cu") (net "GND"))
 (segment (start 133.23 93.23) (end 133.23 94.305) (width 0.2) (layer "F.Cu") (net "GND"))
 (segment (start 129.58 94.305) (end 130.955 92.93) (width 0.2) (layer "F.Cu") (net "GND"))
 (segment (start 121.08 96.305) (end 125.58 96.305) (width 0.2) (layer "F.Cu") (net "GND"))
 (segment (start 132.93 92.93) (end 133.23 93.23) (width 0.2) (layer "F.Cu") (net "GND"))
 (segment (start 146.27 95.525) (end 146.27 98.859448) (width 0.2) (layer "F.Cu") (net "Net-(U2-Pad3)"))
 (segment (start 146.94 103.309448) (end 148.81 105.179448) (width 0.2) (layer "F.Cu") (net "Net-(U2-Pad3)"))
 (segment (start 146.27 98.859448) (end 146.94 99.529448) (width 0.2) (layer "F.Cu") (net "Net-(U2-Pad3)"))
 (segment (start 146.94 99.529448) (end 146.94 103.309448) (width 0.2) (layer "F.Cu") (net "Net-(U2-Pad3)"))
 (segment (start 148.81 105.179448) (end 148.81 105.525) (width 0.2) (layer "F.Cu") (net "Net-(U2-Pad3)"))
 (segment (start 147.54 105.179448) (end 147.54 105.525) (width 0.2) (layer "F.Cu") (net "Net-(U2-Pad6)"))
 (segment (start 142.46 97.589448) (end 144.33 99.459448) (width 0.2) (layer "F.Cu") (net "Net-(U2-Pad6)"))
 (segment (start 144.33 101.969448) (end 147.54 105.179448) (width 0.2) (layer "F.Cu") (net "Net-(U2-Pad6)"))
 (segment (start 142.46 95.525) (end 142.46 97.589448) (width 0.2) (layer "F.Cu") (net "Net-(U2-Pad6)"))
 (segment (start 144.33 99.459448) (end 144.33 101.969448) (width 0.2) (layer "F.Cu") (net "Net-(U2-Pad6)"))
 (segment (start 133.16 109.2) (end 132.08 110.28) (width 0.2) (layer "F.Cu") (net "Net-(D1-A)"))
 (segment (start 146.27 106.499999) (end 143.569999 109.2) (width 0.2) (layer "F.Cu") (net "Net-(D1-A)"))
 (segment (start 146.27 105.525) (end 146.27 106.499999) (width 0.2) (layer "F.Cu") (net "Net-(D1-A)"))
 (segment (start 143.569999 109.2) (end 133.16 109.2) (width 0.2) (layer "F.Cu") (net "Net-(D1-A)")))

